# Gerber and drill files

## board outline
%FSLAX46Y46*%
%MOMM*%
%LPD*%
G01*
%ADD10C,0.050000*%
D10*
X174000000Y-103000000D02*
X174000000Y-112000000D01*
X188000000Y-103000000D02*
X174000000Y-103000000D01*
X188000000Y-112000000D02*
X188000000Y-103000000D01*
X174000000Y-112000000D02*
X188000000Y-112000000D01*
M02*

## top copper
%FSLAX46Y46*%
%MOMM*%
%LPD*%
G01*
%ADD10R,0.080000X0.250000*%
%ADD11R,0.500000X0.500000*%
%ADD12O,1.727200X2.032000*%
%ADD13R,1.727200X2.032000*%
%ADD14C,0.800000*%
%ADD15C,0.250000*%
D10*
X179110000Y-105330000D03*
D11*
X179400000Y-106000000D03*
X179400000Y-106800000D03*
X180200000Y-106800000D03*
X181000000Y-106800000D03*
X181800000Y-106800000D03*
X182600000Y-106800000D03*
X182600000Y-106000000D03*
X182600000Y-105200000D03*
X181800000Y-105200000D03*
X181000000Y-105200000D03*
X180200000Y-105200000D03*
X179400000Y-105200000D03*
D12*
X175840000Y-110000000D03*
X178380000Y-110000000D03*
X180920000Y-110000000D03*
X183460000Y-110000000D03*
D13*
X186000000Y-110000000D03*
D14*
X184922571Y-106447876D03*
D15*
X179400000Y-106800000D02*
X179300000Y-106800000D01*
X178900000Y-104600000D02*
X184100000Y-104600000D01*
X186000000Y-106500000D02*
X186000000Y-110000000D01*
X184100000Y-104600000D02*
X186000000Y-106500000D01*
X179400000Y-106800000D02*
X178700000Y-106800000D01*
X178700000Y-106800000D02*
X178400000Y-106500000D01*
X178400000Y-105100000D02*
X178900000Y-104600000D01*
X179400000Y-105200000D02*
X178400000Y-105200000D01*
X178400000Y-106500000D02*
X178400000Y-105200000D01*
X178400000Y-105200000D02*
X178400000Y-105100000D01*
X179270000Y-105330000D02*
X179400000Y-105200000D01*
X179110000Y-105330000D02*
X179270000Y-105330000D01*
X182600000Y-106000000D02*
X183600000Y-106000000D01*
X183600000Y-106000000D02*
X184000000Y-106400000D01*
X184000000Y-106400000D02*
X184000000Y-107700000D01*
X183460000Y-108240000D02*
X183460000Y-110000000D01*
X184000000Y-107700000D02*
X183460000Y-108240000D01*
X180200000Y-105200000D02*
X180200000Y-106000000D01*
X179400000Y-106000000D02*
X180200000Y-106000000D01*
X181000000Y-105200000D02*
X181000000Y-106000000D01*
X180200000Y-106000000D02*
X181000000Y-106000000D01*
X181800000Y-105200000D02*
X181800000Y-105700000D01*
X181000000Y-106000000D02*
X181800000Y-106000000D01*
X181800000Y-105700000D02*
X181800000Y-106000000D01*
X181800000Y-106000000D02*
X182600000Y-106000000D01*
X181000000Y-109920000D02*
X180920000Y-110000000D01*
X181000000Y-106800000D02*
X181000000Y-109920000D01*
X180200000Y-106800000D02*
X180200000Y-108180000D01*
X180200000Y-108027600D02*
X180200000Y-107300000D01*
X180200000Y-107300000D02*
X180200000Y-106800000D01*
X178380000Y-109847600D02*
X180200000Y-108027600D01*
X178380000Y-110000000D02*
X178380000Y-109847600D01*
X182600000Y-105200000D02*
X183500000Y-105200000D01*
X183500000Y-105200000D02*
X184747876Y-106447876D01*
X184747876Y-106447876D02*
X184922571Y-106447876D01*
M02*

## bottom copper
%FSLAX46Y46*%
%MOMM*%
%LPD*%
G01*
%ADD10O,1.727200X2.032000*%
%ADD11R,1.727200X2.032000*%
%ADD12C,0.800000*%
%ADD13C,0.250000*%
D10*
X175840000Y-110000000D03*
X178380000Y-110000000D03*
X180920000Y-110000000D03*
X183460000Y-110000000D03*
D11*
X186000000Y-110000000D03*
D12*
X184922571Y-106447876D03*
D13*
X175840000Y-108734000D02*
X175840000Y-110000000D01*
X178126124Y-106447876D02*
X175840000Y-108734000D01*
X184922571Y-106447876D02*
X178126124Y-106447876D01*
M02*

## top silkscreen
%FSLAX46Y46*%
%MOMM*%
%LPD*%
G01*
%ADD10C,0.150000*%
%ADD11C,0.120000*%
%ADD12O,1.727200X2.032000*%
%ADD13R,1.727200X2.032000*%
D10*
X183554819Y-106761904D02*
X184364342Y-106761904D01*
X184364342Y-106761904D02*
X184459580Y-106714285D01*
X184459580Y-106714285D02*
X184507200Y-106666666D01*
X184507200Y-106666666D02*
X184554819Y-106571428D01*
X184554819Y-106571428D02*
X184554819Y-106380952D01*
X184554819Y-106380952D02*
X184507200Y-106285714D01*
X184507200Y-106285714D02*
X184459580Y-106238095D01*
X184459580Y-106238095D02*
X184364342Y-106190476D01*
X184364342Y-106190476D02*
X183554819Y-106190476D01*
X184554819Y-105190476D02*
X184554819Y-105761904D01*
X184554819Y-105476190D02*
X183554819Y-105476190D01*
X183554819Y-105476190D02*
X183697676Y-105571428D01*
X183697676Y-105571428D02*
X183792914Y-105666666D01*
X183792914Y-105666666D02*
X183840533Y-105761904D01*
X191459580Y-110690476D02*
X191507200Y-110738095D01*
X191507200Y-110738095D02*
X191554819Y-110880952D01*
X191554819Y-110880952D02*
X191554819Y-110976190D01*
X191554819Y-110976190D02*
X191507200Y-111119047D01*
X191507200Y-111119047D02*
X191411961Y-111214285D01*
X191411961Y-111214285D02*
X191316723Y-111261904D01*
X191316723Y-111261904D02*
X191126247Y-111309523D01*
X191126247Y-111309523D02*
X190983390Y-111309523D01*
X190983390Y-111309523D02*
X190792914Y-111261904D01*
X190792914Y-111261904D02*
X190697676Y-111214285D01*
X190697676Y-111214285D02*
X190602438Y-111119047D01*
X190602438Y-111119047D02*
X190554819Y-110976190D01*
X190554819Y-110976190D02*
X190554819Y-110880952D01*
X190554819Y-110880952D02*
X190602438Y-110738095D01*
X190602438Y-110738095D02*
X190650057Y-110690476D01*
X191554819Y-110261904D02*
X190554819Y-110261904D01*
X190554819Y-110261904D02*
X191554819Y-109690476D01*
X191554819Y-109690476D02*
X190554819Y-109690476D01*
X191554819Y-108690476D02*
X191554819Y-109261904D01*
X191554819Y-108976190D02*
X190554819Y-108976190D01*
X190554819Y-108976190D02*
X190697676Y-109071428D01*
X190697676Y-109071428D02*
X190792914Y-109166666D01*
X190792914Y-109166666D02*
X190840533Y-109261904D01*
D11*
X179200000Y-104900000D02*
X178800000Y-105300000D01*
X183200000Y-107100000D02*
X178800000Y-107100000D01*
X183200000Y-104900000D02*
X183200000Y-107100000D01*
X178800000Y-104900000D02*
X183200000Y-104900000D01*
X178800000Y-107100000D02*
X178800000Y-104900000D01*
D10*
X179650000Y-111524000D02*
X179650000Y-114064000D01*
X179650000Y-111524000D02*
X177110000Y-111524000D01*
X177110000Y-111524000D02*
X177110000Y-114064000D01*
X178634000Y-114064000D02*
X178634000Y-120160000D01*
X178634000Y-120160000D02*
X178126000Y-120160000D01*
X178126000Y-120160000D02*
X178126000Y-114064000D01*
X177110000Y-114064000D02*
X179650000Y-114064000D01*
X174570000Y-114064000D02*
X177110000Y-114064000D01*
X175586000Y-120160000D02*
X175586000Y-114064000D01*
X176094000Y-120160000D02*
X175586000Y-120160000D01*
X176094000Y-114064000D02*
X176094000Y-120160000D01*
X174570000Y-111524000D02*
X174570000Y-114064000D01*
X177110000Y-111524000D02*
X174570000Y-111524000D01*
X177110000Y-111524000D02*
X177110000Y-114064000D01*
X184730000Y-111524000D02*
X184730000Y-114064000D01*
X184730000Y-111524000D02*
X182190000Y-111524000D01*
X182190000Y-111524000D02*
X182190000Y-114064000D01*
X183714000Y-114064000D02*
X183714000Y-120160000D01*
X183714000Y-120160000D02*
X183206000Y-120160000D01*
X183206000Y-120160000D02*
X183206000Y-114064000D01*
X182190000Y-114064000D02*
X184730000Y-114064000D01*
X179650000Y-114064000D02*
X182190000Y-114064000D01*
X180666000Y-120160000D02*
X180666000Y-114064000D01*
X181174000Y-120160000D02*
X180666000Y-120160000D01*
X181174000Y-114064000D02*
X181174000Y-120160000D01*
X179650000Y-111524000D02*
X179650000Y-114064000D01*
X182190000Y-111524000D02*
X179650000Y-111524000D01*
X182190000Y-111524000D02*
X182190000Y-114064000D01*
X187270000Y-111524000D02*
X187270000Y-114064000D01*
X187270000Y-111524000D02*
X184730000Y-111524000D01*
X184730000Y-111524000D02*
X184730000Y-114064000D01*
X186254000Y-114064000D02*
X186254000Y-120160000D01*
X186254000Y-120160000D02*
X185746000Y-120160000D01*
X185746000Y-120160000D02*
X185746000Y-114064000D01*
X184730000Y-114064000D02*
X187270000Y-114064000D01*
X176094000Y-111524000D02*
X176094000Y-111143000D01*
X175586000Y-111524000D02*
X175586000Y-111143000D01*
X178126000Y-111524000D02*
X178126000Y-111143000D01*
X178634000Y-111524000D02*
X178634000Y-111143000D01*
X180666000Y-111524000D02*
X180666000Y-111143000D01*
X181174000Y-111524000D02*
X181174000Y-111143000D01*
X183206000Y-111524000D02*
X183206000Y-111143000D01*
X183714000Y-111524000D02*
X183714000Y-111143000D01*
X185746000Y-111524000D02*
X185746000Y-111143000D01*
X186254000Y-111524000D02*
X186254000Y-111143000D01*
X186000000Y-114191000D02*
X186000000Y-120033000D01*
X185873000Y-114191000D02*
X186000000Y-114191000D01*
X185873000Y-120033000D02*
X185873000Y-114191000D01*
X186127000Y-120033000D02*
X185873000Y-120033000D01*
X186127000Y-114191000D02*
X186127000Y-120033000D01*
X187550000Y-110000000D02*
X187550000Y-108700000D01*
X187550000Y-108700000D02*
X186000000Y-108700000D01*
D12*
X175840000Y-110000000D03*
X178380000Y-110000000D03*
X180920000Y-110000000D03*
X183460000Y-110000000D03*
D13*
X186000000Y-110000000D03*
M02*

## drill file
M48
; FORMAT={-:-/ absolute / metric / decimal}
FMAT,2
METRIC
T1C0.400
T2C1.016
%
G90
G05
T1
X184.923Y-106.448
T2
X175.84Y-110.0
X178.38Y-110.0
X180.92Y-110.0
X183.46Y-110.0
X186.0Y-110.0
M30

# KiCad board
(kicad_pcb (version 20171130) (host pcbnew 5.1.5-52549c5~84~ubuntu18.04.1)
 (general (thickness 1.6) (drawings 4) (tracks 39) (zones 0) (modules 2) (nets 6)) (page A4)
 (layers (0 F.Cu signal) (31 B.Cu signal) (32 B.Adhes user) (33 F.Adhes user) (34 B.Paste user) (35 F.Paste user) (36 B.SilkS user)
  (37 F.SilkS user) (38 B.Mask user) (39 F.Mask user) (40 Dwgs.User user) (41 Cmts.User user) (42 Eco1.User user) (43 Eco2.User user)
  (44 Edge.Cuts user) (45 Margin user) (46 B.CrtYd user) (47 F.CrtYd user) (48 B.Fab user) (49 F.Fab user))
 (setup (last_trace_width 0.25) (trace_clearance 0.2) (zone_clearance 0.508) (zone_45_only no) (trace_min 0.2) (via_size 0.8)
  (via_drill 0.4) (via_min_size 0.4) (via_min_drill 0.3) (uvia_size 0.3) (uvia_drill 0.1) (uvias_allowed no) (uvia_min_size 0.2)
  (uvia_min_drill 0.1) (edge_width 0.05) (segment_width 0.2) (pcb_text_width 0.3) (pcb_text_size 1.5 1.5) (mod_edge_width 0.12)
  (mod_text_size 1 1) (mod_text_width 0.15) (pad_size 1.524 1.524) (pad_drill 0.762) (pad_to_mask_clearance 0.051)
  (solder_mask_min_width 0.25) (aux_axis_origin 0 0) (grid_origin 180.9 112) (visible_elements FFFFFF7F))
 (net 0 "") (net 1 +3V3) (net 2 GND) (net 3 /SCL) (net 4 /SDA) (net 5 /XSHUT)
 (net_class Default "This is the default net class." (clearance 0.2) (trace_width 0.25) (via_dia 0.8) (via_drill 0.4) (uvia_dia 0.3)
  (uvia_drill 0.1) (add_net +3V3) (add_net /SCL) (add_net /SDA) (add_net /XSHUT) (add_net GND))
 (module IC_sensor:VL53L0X (layer F.Cu) (at 181 106 90)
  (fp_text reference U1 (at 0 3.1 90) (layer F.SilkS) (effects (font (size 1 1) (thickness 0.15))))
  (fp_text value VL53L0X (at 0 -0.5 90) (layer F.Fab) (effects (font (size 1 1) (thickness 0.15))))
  (fp_line (start 1.1 -1.8) (end 0.7 -2.2) (layer F.SilkS) (width 0.12))
  (fp_line (start -1.1 2.2) (end -1.1 -2.2) (layer F.SilkS) (width 0.12))
  (fp_line (start 1.1 2.2) (end -1.1 2.2) (layer F.SilkS) (width 0.12))
  (fp_line (start 1.1 -2.2) (end 1.1 2.2) (layer F.SilkS) (width 0.12))
  (fp_line (start -1.1 -2.2) (end 1.1 -2.2) (layer F.SilkS) (width 0.12))
  (pad 1 smd rect (at 0.67 -1.89 90) (size 0.25 0.08) (layers F.Cu F.Paste F.Mask) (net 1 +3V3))
  (pad 12 smd rect (at 0 -1.6 90) (size 0.5 0.5) (layers F.Cu F.Paste F.Mask) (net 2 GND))
  (pad 11 smd rect (at -0.8 -1.6 90) (size 0.5 0.5) (layers F.Cu F.Paste F.Mask) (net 1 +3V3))
  (pad 10 smd rect (at -0.8 -0.8 90) (size 0.5 0.5) (layers F.Cu F.Paste F.Mask) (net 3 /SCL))
  (pad 9 smd rect (at -0.8 0 90) (size 0.5 0.5) (layers F.Cu F.Paste F.Mask) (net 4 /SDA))
  (pad 8 smd rect (at -0.8 0.8 90) (size 0.5 0.5) (layers F.Cu F.Paste F.Mask))
  (pad 7 smd rect (at -0.8 1.6 90) (size 0.5 0.5) (layers F.Cu F.Paste F.Mask))
  (pad 6 smd rect (at 0 1.6 90) (size 0.5 0.5) (layers F.Cu F.Paste F.Mask) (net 2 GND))
  (pad 5 smd rect (at 0.8 1.6 90) (size 0.5 0.5) (layers F.Cu F.Paste F.Mask) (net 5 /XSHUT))
  (pad 4 smd rect (at 0.8 0.8 90) (size 0.5 0.5) (layers F.Cu F.Paste F.Mask) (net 2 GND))
  (pad 3 smd rect (at 0.8 0 90) (size 0.5 0.5) (layers F.Cu F.Paste F.Mask) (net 2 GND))
  (pad 2 smd rect (at 0.8 -0.8 90) (size 0.5 0.5) (layers F.Cu F.Paste F.Mask) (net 2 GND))
  (pad 1 smd rect (at 0.8 -1.6 90) (size 0.5 0.5) (layers F.Cu F.Paste F.Mask) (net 1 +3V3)))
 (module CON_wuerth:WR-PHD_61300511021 (layer F.Cu) (at 186 110 270)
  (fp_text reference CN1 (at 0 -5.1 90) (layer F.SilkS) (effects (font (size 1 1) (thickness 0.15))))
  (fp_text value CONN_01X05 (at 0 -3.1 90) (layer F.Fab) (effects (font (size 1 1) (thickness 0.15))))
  (fp_line (start 1.524 6.35) (end 4.064 6.35) (layer F.SilkS) (width 0.15))
  (fp_line (start 1.524 6.35) (end 1.524 8.89) (layer F.SilkS) (width 0.15))
  (fp_line (start 1.524 8.89) (end 4.064 8.89) (layer F.SilkS) (width 0.15))
  (fp_line (start 4.064 7.366) (end 10.16 7.366) (layer F.SilkS) (width 0.15))
  (fp_line (start 10.16 7.366) (end 10.16 7.874) (layer F.SilkS) (width 0.15))
  (fp_line (start 10.16 7.874) (end 4.064 7.874) (layer F.SilkS) (width 0.15))
  (fp_line (start 4.064 8.89) (end 4.064 6.35) (layer F.SilkS) (width 0.15))
  (fp_line (start 4.064 11.43) (end 4.064 8.89) (layer F.SilkS) (width 0.15))
  (fp_line (start 10.16 10.414) (end 4.064 10.414) (layer F.SilkS) (width 0.15))
  (fp_line (start 10.16 9.906) (end 10.16 10.414) (layer F.SilkS) (width 0.15))
  (fp_line (start 4.064 9.906) (end 10.16 9.906) (layer F.SilkS) (width 0.15))
  (fp_line (start 1.524 11.43) (end 4.064 11.43) (layer F.SilkS) (width 0.15))
  (fp_line (start 1.524 8.89) (end 1.524 11.43) (layer F.SilkS) (width 0.15))
  (fp_line (start 1.524 8.89) (end 4.064 8.89) (layer F.SilkS) (width 0.15))
  (fp_line (start 1.524 1.27) (end 4.064 1.27) (layer F.SilkS) (width 0.15))
  (fp_line (start 1.524 1.27) (end 1.524 3.81) (layer F.SilkS) (width 0.15))
  (fp_line (start 1.524 3.81) (end 4.064 3.81) (layer F.SilkS) (width 0.15))
  (fp_line (start 4.064 2.286) (end 10.16 2.286) (layer F.SilkS) (width 0.15))
  (fp_line (start 10.16 2.286) (end 10.16 2.794) (layer F.SilkS) (width 0.15))
  (fp_line (start 10.16 2.794) (end 4.064 2.794) (layer F.SilkS) (width 0.15))
  (fp_line (start 4.064 3.81) (end 4.064 1.27) (layer F.SilkS) (width 0.15))
  (fp_line (start 4.064 6.35) (end 4.064 3.81) (layer F.SilkS) (width 0.15))
  (fp_line (start 10.16 5.334) (end 4.064 5.334) (layer F.SilkS) (width 0.15))
  (fp_line (start 10.16 4.826) (end 10.16 5.334) (layer F.SilkS) (width 0.15))
  (fp_line (start 4.064 4.826) (end 10.16 4.826) (layer F.SilkS) (width 0.15))
  (fp_line (start 1.524 6.35) (end 4.064 6.35) (layer F.SilkS) (width 0.15))
  (fp_line (start 1.524 3.81) (end 1.524 6.35) (layer F.SilkS) (width 0.15))
  (fp_line (start 1.524 3.81) (end 4.064 3.81) (layer F.SilkS) (width 0.15))
  (fp_line (start 1.524 -1.27) (end 4.064 -1.27) (layer F.SilkS) (width 0.15))
  (fp_line (start 1.524 -1.27) (end 1.524 1.27) (layer F.SilkS) (width 0.15))
  (fp_line (start 1.524 1.27) (end 4.064 1.27) (layer F.SilkS) (width 0.15))
  (fp_line (start 4.064 -0.254) (end 10.16 -0.254) (layer F.SilkS) (width 0.15))
  (fp_line (start 10.16 -0.254) (end 10.16 0.254) (layer F.SilkS) (width 0.15))
  (fp_line (start 10.16 0.254) (end 4.064 0.254) (layer F.SilkS) (width 0.15))
  (fp_line (start 4.064 1.27) (end 4.064 -1.27) (layer F.SilkS) (width 0.15))
  (fp_line (start 1.524 9.906) (end 1.143 9.906) (layer F.SilkS) (width 0.15))
  (fp_line (start 1.524 10.414) (end 1.143 10.414) (layer F.SilkS) (width 0.15))
  (fp_line (start 1.524 7.874) (end 1.143 7.874) (layer F.SilkS) (width 0.15))
  (fp_line (start 1.524 7.366) (end 1.143 7.366) (layer F.SilkS) (width 0.15))
  (fp_line (start 1.524 5.334) (end 1.143 5.334) (layer F.SilkS) (width 0.15))
  (fp_line (start 1.524 4.826) (end 1.143 4.826) (layer F.SilkS) (width 0.15))
  (fp_line (start 1.524 2.794) (end 1.143 2.794) (layer F.SilkS) (width 0.15))
  (fp_line (start 1.524 2.286) (end 1.143 2.286) (layer F.SilkS) (width 0.15))
  (fp_line (start 1.524 0.254) (end 1.143 0.254) (layer F.SilkS) (width 0.15))
  (fp_line (start 1.524 -0.254) (end 1.143 -0.254) (layer F.SilkS) (width 0.15))
  (fp_line (start 4.191 0) (end 10.033 0) (layer F.SilkS) (width 0.15))
  (fp_line (start 4.191 0.127) (end 4.191 0) (layer F.SilkS) (width 0.15))
  (fp_line (start 10.033 0.127) (end 4.191 0.127) (layer F.SilkS) (width 0.15))
  (fp_line (start 10.033 -0.127) (end 10.033 0.127) (layer F.SilkS) (width 0.15))
  (fp_line (start 4.191 -0.127) (end 10.033 -0.127) (layer F.SilkS) (width 0.15))
  (fp_line (start 0 -1.55) (end -1.3 -1.55) (layer F.SilkS) (width 0.15))
  (fp_line (start -1.3 -1.55) (end -1.3 0) (layer F.SilkS) (width 0.15))
  (pad 5 thru_hole oval (at 0 10.16 270) (size 2.032 1.7272) (drill 1.016) (layers *.Cu *.Mask F.SilkS) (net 5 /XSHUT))
  (pad 4 thru_hole oval (at 0 7.62 270) (size 2.032 1.7272) (drill 1.016) (layers *.Cu *.Mask F.SilkS) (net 3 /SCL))
  (pad 3 thru_hole oval (at 0 5.08 270) (size 2.032 1.7272) (drill 1.016) (layers *.Cu *.Mask F.SilkS) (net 4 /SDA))
  (pad 2 thru_hole oval (at 0 2.54 270) (size 2.032 1.7272) (drill 1.016) (layers *.Cu *.Mask F.SilkS) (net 2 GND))
  (pad 1 thru_hole rect (at 0 0 270) (size 2.032 1.7272) (drill 1.016) (layers *.Cu *.Mask F.SilkS) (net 1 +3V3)))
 (gr_line (start 174 103) (end 174 112) (layer Edge.Cuts) (width 0.05))
 (gr_line (start 188 103) (end 174 103) (layer Edge.Cuts) (width 0.05))
 (gr_line (start 188 112) (end 188 103) (layer Edge.Cuts) (width 0.05))
 (gr_line (start 174 112) (end 188 112) (layer Edge.Cuts) (width 0.05))
 (segment (start 179.4 106.8) (end 179.3 106.8) (width 0.25) (layer F.Cu) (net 1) (status 30))
 (segment (start 178.9 104.6) (end 184.1 104.6) (width 0.25) (layer F.Cu) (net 1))
 (segment (start 186 106.5) (end 186 110) (width 0.25) (layer F.Cu) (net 1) (status 20))
 (segment (start 184.1 104.6) (end 186 106.5) (width 0.25) (layer F.Cu) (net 1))
 (segment (start 179.4 106.8) (end 178.7 106.8) (width 0.25) (layer F.Cu) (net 1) (status 10))
 (segment (start 178.7 106.8) (end 178.4 106.5) (width 0.25) (layer F.Cu) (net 1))
 (segment (start 178.4 105.1) (end 178.9 104.6) (width 0.25) (layer F.Cu) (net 1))
 (segment (start 179.4 105.2) (end 178.4 105.2) (width 0.25) (layer F.Cu) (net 1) (status 10))
 (segment (start 178.4 106.5) (end 178.4 105.2) (width 0.25) (layer F.Cu) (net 1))
 (segment (start 178.4 105.2) (end 178.4 105.1) (width 0.25) (layer F.Cu) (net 1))
 (segment (start 179.27 105.33) (end 179.4 105.2) (width 0.25) (layer F.Cu) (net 1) (status 30))
 (segment (start 179.11 105.33) (end 179.27 105.33) (width 0.25) (layer F.Cu) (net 1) (status 30))
 (segment (start 182.6 106) (end 183.6 106) (width 0.25) (layer F.Cu) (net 2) (status 10))
 (segment (start 183.6 106) (end 184 106.4) (width 0.25) (layer F.Cu) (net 2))
 (segment (start 184 106.4) (end 184 107.7) (width 0.25) (layer F.Cu) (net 2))
 (segment (start 183.46 108.24) (end 183.46 110) (width 0.25) (layer F.Cu) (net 2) (status 20))
 (segment (start 184 107.7) (end 183.46 108.24) (width 0.25) (layer F.Cu) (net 2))
 (segment (start 180.2 105.2) (end 180.2 106) (width 0.25) (layer F.Cu) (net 2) (status 10))
 (segment (start 179.4 106) (end 180.2 106) (width 0.25) (layer F.Cu) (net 2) (status 10))
 (segment (start 181 105.2) (end 181 106) (width 0.25) (layer F.Cu) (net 2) (status 10))
 (segment (start 180.2 106) (end 181 106) (width 0.25) (layer F.Cu) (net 2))
 (segment (start 181.8 105.2) (end 181.8 105.7) (width 0.25) (layer F.Cu) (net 2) (status 10))
 (segment (start 181 106) (end 181.8 106) (width 0.25) (layer F.Cu) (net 2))
 (segment (start 181.8 105.7) (end 181.8 106) (width 0.25) (layer F.Cu) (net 2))
 (segment (start 181.8 106) (end 182.6 106) (width 0.25) (layer F.Cu) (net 2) (status 20))
 (segment (start 181 109.92) (end 180.92 110) (width 0.25) (layer F.Cu) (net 4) (status 30))
 (segment (start 181 106.8) (end 181 109.92) (width 0.25) (layer F.Cu) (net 4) (status 30))
 (segment (start 180.2 106.8) (end 180.2 108.18) (width 0.25) (layer F.Cu) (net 3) (status 10))
 (segment (start 180.2 108.0276) (end 180.2 107.3) (width 0.25) (layer F.Cu) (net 3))
 (segment (start 180.2 107.3) (end 180.2 106.8) (width 0.25) (layer F.Cu) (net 3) (status 20))
 (segment (start 178.38 109.8476) (end 180.2 108.0276) (width 0.25) (layer F.Cu) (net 3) (status 10))
 (segment (start 178.38 110) (end 178.38 109.8476) (width 0.25) (layer F.Cu) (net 3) (status 30))
 (segment (start 182.6 105.2) (end 183.5 105.2) (width 0.25) (layer F.Cu) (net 5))
 (via (at 184.922571 106.447876) (size 0.8) (drill 0.4) (layers F.Cu B.Cu) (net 5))
 (segment (start 183.5 105.2) (end 184.747876 106.447876) (width 0.25) (layer F.Cu) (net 5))
 (segment (start 184.747876 106.447876) (end 184.922571 106.447876) (width 0.25) (layer F.Cu) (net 5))
 (segment (start 175.84 108.734) (end 175.84 110) (width 0.25) (layer B.Cu) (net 5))
 (segment (start 178.126124 106.447876) (end 175.84 108.734) (width 0.25) (layer B.Cu) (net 5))
 (segment (start 184.922571 106.447876) (end 178.126124 106.447876) (width 0.25) (layer B.Cu) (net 5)))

